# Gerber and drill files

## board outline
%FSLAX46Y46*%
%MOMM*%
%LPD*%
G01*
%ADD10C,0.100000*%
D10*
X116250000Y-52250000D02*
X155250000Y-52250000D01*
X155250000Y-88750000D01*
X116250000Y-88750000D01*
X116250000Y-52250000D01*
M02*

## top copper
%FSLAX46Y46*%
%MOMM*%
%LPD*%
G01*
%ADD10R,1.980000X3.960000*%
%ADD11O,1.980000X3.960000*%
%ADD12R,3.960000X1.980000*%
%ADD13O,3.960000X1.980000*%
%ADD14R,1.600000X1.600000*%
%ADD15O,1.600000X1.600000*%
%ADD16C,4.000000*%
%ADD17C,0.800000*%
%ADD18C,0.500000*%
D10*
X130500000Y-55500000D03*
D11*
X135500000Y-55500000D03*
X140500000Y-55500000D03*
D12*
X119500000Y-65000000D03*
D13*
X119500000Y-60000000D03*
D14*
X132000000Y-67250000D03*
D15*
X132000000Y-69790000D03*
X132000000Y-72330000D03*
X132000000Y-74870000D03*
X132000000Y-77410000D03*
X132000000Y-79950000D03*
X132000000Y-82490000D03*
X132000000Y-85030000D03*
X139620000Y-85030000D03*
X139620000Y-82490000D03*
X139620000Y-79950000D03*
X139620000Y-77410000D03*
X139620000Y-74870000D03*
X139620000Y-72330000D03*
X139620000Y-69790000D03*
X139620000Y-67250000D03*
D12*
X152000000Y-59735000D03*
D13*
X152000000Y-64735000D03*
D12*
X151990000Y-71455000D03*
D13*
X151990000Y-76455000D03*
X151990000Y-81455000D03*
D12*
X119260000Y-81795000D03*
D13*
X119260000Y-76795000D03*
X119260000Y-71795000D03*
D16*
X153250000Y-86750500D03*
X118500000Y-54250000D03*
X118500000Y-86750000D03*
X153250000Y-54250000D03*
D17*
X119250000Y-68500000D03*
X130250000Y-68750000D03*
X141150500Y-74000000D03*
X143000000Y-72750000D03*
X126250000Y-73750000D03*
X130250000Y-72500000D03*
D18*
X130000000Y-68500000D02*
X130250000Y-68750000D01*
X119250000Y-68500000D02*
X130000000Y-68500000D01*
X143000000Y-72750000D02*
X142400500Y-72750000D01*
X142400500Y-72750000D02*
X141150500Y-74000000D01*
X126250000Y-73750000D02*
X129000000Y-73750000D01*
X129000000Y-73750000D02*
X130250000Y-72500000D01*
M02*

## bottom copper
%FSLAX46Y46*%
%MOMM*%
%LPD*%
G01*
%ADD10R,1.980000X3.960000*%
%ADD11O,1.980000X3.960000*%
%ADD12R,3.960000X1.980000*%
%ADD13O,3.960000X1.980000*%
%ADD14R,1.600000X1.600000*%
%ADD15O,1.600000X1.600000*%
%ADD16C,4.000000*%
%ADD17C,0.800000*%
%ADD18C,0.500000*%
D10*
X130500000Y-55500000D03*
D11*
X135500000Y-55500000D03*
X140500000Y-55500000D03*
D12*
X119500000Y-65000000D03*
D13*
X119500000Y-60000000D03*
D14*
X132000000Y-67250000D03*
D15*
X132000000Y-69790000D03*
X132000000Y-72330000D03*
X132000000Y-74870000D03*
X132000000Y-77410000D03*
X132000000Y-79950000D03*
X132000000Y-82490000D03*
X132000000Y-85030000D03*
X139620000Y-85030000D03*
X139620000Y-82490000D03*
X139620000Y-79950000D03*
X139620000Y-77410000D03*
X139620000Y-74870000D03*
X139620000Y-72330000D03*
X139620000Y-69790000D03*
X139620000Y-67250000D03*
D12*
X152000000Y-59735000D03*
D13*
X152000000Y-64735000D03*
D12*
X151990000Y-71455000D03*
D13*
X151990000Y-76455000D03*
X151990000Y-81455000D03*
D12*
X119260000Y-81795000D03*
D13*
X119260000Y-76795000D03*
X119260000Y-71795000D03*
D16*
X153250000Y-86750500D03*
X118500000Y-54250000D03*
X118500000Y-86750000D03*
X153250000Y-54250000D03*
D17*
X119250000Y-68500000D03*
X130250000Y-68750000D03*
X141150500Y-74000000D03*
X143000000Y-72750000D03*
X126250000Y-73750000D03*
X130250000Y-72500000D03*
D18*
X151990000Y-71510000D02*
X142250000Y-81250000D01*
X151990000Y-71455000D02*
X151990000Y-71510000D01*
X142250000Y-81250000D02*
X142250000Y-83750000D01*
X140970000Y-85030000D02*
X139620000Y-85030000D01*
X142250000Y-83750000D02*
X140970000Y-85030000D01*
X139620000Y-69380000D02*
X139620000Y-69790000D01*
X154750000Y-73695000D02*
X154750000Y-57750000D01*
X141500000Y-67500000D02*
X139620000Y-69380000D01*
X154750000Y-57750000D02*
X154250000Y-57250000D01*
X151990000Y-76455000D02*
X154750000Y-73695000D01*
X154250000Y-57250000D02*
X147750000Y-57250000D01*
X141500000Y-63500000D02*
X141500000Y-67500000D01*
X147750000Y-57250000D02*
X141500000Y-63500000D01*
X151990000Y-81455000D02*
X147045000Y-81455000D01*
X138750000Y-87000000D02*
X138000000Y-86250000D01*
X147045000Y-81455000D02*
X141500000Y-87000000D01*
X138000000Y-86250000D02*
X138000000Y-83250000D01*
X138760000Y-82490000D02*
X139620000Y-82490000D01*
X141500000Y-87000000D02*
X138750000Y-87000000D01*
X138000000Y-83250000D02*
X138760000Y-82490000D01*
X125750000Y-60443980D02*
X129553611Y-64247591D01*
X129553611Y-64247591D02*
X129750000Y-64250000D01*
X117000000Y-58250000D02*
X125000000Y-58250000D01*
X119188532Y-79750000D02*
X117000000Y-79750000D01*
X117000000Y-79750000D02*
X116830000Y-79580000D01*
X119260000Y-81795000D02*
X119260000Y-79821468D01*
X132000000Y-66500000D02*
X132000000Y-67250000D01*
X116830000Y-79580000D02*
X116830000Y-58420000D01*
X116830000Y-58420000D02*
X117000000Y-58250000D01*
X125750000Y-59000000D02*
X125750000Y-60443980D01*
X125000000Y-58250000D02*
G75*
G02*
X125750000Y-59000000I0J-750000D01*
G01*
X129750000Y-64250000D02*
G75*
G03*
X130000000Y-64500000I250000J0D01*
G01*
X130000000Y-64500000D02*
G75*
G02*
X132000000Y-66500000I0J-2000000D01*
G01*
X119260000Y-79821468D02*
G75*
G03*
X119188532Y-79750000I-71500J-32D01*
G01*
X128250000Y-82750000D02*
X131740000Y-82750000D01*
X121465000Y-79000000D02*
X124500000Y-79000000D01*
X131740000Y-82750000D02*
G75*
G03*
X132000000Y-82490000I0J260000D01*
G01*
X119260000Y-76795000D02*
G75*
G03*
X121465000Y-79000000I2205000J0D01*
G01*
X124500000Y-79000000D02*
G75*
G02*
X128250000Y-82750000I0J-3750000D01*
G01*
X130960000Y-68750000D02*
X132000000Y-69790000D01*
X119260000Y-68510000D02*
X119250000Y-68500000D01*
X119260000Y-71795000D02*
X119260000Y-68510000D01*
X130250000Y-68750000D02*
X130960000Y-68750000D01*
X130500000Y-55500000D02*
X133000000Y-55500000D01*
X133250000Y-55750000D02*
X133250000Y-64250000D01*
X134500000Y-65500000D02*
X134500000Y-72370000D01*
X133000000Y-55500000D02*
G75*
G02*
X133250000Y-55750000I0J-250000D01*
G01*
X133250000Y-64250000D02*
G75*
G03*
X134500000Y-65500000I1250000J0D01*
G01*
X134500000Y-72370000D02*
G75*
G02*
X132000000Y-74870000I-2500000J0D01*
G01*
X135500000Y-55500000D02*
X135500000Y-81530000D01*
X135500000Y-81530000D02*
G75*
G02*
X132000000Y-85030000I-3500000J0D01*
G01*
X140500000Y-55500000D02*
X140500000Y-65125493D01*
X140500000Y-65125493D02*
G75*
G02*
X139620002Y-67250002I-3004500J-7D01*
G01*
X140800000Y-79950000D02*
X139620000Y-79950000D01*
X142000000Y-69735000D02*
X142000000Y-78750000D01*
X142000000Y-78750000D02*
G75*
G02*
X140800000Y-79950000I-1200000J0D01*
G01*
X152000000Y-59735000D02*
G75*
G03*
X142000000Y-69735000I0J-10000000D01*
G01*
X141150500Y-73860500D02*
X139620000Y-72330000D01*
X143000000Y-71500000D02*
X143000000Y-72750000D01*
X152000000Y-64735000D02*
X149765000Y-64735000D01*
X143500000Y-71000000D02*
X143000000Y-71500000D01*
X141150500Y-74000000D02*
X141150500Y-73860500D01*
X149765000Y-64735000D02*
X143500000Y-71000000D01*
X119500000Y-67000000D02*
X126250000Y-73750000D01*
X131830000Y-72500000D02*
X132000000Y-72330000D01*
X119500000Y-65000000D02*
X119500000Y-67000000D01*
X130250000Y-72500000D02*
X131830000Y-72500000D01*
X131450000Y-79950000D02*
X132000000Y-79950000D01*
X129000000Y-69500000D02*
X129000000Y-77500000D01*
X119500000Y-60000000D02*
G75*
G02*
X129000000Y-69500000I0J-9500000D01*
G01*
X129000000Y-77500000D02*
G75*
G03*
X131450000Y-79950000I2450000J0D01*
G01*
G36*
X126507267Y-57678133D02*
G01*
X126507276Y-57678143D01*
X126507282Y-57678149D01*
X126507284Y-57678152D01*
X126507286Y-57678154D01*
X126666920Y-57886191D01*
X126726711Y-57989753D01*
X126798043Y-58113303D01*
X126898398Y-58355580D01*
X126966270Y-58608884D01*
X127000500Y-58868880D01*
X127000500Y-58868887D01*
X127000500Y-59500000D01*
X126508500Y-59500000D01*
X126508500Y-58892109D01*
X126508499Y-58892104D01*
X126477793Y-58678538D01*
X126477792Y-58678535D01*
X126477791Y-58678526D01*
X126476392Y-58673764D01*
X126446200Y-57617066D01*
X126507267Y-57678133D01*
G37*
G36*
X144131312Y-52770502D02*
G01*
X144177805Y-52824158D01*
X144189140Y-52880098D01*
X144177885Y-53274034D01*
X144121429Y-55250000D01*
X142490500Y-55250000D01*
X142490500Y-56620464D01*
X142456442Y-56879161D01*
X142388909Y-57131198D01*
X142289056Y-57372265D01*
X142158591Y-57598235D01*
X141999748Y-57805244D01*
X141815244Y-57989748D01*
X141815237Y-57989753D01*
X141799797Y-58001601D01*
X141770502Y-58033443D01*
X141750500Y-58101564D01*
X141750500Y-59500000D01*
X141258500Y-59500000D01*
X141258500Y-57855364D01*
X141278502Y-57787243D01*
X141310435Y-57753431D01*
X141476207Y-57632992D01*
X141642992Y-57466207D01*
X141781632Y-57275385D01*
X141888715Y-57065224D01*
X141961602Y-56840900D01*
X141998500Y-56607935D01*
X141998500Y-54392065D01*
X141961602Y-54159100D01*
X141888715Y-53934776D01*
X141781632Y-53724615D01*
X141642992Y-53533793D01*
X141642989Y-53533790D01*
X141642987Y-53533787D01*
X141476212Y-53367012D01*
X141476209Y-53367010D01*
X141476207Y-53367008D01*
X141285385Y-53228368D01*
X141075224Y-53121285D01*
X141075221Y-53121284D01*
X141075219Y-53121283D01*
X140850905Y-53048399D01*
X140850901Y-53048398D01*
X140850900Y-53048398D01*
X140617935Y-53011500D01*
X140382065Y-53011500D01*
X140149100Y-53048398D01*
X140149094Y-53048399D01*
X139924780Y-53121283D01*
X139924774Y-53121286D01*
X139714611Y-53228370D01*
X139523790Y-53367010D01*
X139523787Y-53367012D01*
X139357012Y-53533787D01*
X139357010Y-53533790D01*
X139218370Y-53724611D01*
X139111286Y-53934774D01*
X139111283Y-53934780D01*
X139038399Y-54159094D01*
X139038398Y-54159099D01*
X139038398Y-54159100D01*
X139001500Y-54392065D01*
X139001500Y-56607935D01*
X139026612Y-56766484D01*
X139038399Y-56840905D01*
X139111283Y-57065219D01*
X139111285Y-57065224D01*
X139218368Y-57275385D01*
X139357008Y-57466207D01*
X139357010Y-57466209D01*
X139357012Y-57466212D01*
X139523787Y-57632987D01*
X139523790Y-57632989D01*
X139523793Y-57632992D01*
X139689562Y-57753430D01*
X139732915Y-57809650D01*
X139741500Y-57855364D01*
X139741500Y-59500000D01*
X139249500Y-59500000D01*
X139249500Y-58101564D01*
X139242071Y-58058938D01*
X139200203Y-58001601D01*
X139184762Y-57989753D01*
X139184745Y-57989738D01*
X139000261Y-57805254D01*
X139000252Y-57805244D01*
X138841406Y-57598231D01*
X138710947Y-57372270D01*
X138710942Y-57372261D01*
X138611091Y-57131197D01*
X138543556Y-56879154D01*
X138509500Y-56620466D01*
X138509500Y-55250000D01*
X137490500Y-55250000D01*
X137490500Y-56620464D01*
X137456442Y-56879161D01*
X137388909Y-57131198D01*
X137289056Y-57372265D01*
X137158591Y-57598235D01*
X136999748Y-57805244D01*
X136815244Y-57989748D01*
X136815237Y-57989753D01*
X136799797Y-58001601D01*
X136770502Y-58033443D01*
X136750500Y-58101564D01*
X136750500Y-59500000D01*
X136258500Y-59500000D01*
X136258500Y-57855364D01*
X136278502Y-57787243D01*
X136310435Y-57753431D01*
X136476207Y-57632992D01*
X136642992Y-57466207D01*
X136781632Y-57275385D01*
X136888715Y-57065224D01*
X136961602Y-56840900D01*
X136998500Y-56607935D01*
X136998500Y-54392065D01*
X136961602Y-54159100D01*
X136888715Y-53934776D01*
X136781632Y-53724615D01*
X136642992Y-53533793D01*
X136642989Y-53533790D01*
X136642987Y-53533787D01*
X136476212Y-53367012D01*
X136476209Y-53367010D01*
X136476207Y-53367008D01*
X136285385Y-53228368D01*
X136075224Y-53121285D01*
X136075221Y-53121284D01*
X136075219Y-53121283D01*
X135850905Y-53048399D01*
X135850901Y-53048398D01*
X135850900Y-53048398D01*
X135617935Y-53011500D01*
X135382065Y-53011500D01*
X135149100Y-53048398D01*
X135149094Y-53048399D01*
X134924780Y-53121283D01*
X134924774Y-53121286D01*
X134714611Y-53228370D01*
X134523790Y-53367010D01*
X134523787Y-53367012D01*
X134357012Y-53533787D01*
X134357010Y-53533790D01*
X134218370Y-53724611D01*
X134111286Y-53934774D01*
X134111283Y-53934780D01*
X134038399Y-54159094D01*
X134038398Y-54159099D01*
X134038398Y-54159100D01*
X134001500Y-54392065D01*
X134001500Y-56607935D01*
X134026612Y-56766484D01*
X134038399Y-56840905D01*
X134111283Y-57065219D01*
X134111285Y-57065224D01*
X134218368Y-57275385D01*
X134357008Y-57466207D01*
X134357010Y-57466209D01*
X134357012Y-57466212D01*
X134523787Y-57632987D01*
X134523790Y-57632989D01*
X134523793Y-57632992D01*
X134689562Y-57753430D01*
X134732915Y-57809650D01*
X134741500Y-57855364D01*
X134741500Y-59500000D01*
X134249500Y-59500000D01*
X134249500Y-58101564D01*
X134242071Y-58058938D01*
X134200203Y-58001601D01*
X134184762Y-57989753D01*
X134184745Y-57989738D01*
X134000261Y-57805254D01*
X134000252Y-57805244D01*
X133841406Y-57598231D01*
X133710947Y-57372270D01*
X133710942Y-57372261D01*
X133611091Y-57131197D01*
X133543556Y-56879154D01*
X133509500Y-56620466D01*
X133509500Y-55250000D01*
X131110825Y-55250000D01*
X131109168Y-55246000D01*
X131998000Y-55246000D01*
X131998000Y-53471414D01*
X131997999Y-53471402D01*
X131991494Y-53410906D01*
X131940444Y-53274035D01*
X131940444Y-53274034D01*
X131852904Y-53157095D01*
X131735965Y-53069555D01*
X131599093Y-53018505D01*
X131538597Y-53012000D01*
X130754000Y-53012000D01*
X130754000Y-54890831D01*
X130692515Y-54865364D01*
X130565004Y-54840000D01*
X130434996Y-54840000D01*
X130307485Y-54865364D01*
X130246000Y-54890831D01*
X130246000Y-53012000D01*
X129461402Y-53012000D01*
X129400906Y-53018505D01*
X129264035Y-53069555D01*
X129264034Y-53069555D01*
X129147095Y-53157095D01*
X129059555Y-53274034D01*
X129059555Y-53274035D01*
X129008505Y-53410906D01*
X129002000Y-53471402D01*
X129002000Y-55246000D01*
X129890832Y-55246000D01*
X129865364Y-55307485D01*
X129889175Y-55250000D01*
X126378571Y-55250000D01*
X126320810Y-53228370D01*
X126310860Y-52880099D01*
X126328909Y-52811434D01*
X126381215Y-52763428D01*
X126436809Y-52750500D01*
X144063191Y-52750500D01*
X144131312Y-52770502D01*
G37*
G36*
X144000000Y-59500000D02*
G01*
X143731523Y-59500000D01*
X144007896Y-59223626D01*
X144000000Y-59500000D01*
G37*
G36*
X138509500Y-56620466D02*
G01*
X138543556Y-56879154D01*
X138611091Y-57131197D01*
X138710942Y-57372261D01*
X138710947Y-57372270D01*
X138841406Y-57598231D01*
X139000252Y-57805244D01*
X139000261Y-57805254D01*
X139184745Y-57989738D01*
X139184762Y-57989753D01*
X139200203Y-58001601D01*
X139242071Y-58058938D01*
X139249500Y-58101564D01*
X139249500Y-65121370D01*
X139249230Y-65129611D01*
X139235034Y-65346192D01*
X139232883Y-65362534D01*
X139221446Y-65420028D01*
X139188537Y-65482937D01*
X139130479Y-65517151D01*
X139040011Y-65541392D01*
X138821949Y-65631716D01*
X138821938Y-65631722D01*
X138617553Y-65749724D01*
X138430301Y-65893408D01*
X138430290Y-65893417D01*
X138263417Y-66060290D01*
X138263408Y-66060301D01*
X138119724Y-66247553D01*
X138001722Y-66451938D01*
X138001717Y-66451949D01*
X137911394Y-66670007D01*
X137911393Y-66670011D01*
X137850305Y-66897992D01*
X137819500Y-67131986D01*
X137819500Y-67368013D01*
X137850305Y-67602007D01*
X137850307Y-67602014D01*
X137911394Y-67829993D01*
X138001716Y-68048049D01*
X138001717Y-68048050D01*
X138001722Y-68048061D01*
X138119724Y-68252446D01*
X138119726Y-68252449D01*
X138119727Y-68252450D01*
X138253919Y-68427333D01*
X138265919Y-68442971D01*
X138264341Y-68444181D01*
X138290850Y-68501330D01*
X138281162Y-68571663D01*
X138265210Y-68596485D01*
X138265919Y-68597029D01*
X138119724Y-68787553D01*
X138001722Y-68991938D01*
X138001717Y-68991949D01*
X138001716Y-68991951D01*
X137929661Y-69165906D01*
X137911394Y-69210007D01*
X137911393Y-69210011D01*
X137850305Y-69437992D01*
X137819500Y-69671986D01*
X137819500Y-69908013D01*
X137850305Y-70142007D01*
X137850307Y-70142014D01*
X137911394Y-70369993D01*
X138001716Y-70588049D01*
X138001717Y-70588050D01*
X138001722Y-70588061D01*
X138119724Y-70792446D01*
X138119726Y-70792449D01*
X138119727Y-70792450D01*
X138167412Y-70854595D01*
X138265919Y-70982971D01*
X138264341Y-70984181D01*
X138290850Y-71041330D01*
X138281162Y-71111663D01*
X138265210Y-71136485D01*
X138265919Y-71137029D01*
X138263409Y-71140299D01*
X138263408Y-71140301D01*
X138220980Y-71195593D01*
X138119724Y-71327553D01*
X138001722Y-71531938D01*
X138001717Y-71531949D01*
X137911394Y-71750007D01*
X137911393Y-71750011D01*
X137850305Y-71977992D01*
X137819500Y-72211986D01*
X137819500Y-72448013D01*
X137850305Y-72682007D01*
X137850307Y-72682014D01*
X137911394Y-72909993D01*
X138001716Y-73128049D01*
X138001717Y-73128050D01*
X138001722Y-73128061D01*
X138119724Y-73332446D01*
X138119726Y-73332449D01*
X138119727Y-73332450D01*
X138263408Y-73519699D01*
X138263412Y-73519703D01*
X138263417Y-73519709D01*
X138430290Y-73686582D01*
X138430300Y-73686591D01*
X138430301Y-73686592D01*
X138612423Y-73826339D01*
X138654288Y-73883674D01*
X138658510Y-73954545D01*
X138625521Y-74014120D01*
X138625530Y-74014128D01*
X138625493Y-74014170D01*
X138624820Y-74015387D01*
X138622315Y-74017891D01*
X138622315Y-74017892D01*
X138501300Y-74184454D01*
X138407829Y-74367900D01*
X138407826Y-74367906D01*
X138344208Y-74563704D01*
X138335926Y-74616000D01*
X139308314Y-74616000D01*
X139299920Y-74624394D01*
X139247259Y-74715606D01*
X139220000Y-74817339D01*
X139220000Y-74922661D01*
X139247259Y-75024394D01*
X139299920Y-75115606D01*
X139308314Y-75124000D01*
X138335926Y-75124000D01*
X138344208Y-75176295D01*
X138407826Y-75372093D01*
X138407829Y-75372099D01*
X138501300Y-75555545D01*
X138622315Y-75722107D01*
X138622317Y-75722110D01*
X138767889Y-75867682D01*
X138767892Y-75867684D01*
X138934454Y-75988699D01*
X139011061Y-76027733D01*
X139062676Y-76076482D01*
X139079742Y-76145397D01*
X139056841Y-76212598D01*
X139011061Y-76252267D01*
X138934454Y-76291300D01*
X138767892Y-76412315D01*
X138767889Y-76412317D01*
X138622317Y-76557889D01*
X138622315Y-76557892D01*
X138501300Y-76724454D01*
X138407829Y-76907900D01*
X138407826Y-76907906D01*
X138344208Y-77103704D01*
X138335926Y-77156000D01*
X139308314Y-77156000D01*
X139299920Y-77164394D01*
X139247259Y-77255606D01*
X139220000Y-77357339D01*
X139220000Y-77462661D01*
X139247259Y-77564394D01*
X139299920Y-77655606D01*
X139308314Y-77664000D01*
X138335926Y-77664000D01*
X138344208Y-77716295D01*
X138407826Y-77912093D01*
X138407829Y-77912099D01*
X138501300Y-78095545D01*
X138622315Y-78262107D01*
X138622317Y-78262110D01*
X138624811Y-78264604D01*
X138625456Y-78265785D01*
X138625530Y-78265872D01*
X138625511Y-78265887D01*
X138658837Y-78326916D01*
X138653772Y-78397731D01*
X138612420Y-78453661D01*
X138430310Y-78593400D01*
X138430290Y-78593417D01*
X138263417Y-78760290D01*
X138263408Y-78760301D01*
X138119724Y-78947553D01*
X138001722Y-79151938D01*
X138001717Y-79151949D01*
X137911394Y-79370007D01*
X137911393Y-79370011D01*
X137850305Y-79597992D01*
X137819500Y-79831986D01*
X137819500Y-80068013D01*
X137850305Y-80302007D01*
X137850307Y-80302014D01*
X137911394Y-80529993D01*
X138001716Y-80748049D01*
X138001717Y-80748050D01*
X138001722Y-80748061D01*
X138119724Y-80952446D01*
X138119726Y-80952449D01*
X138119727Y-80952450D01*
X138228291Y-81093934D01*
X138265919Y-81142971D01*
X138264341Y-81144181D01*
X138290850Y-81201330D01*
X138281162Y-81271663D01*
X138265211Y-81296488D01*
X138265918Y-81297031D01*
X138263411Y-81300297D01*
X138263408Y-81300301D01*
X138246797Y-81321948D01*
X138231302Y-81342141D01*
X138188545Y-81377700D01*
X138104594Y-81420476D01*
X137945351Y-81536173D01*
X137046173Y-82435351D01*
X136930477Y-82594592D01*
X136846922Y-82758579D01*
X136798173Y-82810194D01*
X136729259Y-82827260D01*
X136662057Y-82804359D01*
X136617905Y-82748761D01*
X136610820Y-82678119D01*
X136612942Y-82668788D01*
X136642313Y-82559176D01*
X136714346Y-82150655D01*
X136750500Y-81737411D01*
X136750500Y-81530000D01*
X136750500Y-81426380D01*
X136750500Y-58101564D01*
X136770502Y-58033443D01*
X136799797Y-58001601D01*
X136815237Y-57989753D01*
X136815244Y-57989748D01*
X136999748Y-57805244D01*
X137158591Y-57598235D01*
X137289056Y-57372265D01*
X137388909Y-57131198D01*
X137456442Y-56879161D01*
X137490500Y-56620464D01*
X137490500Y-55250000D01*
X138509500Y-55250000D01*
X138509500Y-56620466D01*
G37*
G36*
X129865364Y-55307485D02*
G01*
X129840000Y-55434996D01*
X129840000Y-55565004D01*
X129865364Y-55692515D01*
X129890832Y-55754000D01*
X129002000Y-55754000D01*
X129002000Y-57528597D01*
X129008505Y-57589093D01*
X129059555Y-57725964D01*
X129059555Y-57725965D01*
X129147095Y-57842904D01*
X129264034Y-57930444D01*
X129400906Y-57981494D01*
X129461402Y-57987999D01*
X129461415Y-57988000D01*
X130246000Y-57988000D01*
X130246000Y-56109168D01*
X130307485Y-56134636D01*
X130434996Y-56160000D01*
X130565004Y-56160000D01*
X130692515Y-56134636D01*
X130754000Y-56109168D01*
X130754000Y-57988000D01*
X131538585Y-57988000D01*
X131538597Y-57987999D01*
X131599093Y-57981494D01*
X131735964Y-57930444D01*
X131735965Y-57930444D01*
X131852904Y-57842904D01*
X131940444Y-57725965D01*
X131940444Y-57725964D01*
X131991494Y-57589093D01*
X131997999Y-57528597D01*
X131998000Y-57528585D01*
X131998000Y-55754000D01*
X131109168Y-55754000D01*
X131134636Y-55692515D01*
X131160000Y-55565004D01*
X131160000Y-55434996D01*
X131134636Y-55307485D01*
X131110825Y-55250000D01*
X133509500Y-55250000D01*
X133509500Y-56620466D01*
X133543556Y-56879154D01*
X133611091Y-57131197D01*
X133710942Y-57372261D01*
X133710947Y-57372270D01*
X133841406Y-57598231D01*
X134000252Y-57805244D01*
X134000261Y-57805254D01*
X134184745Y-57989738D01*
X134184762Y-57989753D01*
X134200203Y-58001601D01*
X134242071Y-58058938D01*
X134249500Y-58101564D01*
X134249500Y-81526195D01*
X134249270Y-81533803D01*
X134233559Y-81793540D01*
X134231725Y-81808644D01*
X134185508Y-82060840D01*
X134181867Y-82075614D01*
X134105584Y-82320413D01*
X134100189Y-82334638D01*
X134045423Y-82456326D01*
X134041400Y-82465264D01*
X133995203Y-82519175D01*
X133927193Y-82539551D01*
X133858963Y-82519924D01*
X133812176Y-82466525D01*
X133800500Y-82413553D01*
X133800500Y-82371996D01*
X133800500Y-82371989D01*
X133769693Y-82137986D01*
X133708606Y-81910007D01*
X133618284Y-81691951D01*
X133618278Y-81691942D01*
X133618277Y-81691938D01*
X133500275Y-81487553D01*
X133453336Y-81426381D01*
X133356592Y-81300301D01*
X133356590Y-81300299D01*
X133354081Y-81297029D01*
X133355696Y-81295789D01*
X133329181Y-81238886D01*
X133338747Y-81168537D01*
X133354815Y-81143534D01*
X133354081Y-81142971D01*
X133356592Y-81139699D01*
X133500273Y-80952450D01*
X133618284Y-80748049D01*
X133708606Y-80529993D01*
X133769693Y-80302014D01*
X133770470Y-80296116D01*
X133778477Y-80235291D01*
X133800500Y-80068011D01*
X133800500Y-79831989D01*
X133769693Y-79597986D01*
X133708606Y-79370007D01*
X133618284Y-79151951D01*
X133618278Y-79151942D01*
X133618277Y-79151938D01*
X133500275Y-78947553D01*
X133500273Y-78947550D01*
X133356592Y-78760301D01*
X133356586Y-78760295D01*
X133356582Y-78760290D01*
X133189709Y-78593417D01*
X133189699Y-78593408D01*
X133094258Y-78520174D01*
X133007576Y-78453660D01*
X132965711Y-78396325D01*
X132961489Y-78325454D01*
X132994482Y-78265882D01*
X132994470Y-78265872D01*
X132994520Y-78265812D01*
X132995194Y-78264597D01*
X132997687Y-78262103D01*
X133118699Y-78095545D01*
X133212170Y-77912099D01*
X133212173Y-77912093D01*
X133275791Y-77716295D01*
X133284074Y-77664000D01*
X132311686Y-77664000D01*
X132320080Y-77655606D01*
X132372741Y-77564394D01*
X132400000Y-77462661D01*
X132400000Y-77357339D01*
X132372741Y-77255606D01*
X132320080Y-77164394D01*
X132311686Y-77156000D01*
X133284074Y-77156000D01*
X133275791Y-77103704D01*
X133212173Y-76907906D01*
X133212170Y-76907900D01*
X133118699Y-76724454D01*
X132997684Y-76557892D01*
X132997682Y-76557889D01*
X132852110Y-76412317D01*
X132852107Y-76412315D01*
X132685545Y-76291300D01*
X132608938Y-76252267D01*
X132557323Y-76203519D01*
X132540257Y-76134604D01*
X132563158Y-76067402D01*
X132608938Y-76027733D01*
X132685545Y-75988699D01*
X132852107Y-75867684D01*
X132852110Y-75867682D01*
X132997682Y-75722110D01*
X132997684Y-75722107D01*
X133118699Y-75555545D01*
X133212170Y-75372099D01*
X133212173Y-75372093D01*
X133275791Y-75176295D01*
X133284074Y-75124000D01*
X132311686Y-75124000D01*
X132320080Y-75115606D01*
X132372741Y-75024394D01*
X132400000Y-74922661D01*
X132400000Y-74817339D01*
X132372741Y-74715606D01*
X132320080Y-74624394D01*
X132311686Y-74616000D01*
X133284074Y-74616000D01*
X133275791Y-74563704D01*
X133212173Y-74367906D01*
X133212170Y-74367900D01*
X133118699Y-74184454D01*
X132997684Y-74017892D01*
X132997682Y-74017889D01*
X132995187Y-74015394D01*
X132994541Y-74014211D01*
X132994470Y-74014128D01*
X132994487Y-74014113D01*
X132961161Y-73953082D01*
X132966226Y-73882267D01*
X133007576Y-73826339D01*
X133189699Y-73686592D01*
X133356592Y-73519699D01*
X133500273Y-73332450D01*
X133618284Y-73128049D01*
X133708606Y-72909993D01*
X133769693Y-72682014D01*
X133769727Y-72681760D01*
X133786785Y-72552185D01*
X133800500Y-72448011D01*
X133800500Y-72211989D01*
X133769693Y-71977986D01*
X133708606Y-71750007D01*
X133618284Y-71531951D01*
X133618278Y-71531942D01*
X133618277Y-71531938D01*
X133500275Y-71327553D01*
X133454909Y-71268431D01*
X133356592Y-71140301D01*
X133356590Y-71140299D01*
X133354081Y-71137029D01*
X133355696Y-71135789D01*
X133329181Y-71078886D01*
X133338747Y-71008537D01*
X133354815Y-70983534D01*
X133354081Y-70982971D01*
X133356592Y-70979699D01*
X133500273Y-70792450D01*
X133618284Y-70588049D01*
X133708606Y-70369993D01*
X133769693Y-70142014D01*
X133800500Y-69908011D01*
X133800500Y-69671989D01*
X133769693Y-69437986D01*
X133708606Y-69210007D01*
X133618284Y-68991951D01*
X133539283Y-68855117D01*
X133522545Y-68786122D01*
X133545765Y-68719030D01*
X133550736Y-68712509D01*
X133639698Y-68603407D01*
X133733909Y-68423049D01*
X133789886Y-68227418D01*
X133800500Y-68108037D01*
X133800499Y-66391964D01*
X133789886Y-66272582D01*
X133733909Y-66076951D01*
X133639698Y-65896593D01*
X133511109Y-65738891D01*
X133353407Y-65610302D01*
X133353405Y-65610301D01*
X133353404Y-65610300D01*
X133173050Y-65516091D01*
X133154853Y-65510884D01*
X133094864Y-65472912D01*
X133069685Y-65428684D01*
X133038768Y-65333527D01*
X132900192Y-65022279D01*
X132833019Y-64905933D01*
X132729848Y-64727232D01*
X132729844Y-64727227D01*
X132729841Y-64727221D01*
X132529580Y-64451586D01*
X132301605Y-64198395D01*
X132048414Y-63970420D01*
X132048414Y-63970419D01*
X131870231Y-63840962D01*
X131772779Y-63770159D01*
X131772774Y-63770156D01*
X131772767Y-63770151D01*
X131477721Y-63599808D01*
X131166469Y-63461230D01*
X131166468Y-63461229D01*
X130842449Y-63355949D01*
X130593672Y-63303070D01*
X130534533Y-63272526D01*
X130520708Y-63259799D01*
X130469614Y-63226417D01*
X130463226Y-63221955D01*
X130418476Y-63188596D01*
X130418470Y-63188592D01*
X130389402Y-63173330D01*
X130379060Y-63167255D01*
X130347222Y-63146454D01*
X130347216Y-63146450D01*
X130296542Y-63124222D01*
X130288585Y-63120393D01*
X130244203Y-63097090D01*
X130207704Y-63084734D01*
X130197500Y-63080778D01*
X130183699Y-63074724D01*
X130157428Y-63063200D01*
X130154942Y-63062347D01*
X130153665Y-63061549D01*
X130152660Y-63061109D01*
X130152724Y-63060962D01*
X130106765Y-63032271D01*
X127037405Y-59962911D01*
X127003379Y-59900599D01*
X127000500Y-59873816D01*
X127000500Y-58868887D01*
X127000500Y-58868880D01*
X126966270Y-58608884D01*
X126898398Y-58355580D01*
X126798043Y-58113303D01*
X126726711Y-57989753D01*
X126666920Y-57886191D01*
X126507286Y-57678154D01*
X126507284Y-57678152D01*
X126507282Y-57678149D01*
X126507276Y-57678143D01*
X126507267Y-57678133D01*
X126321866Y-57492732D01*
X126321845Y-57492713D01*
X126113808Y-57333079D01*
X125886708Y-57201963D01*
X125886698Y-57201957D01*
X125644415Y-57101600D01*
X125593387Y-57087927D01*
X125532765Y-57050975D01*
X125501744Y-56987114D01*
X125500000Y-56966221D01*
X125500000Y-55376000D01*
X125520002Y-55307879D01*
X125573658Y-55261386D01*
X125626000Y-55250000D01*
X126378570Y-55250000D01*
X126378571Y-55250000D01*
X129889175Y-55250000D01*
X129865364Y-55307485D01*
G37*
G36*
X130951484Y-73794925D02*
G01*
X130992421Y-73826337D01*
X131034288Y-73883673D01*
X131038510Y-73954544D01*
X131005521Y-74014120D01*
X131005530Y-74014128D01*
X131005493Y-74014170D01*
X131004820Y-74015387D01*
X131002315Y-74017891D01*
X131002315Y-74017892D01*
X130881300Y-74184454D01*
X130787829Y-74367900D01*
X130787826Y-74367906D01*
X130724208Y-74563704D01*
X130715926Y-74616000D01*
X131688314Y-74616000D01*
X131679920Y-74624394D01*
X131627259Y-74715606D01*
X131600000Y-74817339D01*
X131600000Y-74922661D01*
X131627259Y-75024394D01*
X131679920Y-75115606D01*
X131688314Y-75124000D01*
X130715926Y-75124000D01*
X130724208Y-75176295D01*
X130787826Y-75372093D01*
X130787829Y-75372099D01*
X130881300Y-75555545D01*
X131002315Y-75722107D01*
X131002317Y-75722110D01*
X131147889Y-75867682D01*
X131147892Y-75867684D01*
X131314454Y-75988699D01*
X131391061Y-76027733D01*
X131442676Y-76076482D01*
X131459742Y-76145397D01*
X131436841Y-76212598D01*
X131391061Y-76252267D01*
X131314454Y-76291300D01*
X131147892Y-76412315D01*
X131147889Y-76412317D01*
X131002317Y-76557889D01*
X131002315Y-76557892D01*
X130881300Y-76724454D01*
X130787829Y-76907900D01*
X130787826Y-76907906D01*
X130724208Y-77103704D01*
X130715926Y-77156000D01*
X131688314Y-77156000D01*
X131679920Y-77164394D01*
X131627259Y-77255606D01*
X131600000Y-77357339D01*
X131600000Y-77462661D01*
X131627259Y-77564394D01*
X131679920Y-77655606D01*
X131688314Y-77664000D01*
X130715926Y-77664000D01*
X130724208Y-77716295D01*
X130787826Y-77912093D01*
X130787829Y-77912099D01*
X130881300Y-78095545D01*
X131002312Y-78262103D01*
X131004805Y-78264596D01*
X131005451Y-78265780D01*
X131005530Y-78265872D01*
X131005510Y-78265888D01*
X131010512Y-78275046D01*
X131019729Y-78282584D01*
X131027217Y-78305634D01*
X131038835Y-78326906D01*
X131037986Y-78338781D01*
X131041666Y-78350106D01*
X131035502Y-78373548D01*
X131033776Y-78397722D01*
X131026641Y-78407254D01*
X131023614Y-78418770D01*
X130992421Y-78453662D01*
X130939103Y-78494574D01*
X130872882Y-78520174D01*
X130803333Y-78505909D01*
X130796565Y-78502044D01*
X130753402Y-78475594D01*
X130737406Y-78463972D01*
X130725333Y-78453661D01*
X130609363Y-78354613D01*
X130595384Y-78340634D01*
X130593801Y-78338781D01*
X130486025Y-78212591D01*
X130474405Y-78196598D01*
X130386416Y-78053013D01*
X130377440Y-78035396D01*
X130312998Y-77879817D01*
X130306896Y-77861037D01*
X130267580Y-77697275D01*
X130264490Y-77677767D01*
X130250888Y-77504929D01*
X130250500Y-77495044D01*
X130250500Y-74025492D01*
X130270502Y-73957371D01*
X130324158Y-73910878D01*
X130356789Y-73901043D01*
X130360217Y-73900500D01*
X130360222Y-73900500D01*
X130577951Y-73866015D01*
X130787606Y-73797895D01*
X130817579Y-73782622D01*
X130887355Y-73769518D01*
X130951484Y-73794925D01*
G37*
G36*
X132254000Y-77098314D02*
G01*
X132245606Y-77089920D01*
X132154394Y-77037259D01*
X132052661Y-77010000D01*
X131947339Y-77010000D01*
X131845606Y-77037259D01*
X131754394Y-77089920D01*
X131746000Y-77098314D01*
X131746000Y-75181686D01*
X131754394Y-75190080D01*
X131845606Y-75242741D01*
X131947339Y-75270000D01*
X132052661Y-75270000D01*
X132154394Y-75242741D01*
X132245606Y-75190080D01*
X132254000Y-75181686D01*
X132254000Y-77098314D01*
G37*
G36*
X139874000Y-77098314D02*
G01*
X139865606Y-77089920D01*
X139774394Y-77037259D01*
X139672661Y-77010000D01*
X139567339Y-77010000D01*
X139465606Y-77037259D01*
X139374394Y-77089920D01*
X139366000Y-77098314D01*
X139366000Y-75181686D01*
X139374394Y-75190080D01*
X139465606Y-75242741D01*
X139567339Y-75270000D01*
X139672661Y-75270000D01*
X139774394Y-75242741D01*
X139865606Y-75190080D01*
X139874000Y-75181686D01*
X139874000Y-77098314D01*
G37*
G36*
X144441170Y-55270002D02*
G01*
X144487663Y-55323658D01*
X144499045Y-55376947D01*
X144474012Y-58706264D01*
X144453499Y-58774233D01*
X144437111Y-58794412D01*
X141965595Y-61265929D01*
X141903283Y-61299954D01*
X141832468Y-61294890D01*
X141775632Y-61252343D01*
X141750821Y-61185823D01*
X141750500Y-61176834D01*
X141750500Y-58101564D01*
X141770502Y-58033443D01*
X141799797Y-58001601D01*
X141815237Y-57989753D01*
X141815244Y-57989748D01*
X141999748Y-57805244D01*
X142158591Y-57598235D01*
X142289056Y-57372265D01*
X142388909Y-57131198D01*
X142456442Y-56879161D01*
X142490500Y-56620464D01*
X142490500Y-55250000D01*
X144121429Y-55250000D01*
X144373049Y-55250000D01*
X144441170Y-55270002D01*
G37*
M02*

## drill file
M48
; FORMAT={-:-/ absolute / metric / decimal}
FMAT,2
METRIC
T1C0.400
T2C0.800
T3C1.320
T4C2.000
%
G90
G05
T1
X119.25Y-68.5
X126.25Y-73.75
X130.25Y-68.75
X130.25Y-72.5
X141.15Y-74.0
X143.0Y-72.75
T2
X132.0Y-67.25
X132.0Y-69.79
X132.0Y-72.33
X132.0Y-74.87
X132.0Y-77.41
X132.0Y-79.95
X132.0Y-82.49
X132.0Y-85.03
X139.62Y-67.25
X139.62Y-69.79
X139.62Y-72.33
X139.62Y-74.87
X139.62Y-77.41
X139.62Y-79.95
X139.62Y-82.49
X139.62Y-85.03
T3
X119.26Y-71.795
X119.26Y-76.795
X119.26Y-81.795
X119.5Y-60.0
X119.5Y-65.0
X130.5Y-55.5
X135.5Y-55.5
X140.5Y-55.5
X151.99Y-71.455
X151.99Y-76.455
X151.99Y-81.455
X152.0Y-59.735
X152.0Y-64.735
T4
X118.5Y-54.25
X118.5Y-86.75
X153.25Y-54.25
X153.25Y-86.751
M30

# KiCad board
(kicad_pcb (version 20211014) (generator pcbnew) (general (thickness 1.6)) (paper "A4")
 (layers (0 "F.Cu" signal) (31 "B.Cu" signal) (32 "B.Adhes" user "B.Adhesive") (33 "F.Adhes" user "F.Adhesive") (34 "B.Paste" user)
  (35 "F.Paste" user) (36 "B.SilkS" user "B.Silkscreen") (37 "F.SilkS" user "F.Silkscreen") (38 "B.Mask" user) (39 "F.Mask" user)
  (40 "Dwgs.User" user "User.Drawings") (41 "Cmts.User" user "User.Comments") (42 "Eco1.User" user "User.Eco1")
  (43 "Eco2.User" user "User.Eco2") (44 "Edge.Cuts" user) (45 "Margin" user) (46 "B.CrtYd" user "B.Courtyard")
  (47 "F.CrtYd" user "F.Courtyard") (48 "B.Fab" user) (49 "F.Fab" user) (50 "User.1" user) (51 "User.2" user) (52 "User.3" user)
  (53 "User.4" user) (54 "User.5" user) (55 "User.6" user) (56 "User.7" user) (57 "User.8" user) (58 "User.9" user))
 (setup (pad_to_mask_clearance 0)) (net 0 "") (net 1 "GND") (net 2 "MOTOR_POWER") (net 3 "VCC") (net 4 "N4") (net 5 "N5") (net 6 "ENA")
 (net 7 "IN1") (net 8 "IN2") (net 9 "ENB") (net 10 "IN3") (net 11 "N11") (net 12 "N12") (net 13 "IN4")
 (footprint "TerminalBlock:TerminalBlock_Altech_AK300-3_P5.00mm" (layer "F.Cu") (at 130.5 55.5)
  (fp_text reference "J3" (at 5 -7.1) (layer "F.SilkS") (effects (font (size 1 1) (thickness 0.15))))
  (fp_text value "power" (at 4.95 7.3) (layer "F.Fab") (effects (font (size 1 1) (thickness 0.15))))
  (pad "1" thru_hole rect (at 0 0) (size 1.98 3.96) (drill 1.32) (layers *.Cu *.Mask) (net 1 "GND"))
  (pad "2" thru_hole oval (at 5 0) (size 1.98 3.96) (drill 1.32) (layers *.Cu *.Mask) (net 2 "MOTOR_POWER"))
  (pad "3" thru_hole oval (at 10 0) (size 1.98 3.96) (drill 1.32) (layers *.Cu *.Mask) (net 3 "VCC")))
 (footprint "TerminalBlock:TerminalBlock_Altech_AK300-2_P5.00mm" (layer "F.Cu") (at 119.5 65 90)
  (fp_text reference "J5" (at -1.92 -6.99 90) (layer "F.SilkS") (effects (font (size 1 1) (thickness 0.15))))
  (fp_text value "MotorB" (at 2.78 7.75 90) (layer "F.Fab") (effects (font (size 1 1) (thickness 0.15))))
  (pad "1" thru_hole rect (at 0 0 90) (size 1.98 3.96) (drill 1.32) (layers *.Cu *.Mask) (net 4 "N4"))
  (pad "2" thru_hole oval (at 5 0 90) (size 1.98 3.96) (drill 1.32) (layers *.Cu *.Mask) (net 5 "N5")))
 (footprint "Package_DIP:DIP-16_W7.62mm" (layer "F.Cu") (at 132 67.25)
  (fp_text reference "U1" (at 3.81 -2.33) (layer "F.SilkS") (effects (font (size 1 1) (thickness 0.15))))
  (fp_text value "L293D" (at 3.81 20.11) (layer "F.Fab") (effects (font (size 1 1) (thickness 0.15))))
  (pad "1" thru_hole rect (at 0 0) (size 1.6 1.6) (drill 0.8) (layers *.Cu *.Mask) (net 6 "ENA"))
  (pad "2" thru_hole oval (at 0 2.54) (size 1.6 1.6) (drill 0.8) (layers *.Cu *.Mask) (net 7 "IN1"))
  (pad "3" thru_hole oval (at 0 5.08) (size 1.6 1.6) (drill 0.8) (layers *.Cu *.Mask) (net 4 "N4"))
  (pad "4" thru_hole oval (at 0 7.62) (size 1.6 1.6) (drill 0.8) (layers *.Cu *.Mask) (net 1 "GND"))
  (pad "5" thru_hole oval (at 0 10.16) (size 1.6 1.6) (drill 0.8) (layers *.Cu *.Mask) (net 1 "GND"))
  (pad "6" thru_hole oval (at 0 12.7) (size 1.6 1.6) (drill 0.8) (layers *.Cu *.Mask) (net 5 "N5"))
  (pad "7" thru_hole oval (at 0 15.24) (size 1.6 1.6) (drill 0.8) (layers *.Cu *.Mask) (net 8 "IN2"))
  (pad "8" thru_hole oval (at 0 17.78) (size 1.6 1.6) (drill 0.8) (layers *.Cu *.Mask) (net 2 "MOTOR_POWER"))
  (pad "9" thru_hole oval (at 7.62 17.78) (size 1.6 1.6) (drill 0.8) (layers *.Cu *.Mask) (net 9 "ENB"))
  (pad "10" thru_hole oval (at 7.62 15.24) (size 1.6 1.6) (drill 0.8) (layers *.Cu *.Mask) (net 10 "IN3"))
  (pad "11" thru_hole oval (at 7.62 12.7) (size 1.6 1.6) (drill 0.8) (layers *.Cu *.Mask) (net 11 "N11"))
  (pad "12" thru_hole oval (at 7.62 10.16) (size 1.6 1.6) (drill 0.8) (layers *.Cu *.Mask) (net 1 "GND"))
  (pad "13" thru_hole oval (at 7.62 7.62) (size 1.6 1.6) (drill 0.8) (layers *.Cu *.Mask) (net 1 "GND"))
  (pad "14" thru_hole oval (at 7.62 5.08) (size 1.6 1.6) (drill 0.8) (layers *.Cu *.Mask) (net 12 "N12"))
  (pad "15" thru_hole oval (at 7.62 2.54) (size 1.6 1.6) (drill 0.8) (layers *.Cu *.Mask) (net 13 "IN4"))
  (pad "16" thru_hole oval (at 7.62 0) (size 1.6 1.6) (drill 0.8) (layers *.Cu *.Mask) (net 3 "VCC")))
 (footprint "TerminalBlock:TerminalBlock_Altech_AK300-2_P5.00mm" (layer "F.Cu") (at 152 59.735 -90)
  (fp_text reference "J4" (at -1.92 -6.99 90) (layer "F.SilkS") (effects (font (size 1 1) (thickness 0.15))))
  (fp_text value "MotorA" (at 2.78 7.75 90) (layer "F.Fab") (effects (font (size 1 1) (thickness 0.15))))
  (pad "1" thru_hole rect (at 0 0 270) (size 1.98 3.96) (drill 1.32) (layers *.Cu *.Mask) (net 11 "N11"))
  (pad "2" thru_hole oval (at 5 0 270) (size 1.98 3.96) (drill 1.32) (layers *.Cu *.Mask) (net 12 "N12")))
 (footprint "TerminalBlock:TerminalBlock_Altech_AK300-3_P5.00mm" (layer "F.Cu") (at 151.99 71.455 -90)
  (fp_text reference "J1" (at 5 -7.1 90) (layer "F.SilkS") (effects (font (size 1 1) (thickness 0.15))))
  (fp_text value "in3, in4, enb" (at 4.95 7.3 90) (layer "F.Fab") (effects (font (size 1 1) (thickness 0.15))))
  (pad "1" thru_hole rect (at 0 0 270) (size 1.98 3.96) (drill 1.32) (layers *.Cu *.Mask) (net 9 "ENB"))
  (pad "2" thru_hole oval (at 5 0 270) (size 1.98 3.96) (drill 1.32) (layers *.Cu *.Mask) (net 13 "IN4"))
  (pad "3" thru_hole oval (at 10 0 270) (size 1.98 3.96) (drill 1.32) (layers *.Cu *.Mask) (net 10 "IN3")))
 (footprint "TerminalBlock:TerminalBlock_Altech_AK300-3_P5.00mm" (layer "F.Cu") (at 119.26 81.795 90)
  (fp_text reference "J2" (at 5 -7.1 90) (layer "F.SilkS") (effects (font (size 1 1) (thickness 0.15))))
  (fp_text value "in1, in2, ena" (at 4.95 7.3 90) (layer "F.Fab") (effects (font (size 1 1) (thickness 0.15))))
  (pad "1" thru_hole rect (at 0 0 90) (size 1.98 3.96) (drill 1.32) (layers *.Cu *.Mask) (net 6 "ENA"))
  (pad "2" thru_hole oval (at 5 0 90) (size 1.98 3.96) (drill 1.32) (layers *.Cu *.Mask) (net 8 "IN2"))
  (pad "3" thru_hole oval (at 10 0 90) (size 1.98 3.96) (drill 1.32) (layers *.Cu *.Mask) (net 7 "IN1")))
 (gr_rect (start 116.25 52.25) (end 155.25 88.75) (layer "Edge.Cuts") (width 0.1) (fill none))
 (via (at 153.25 86.7505) (size 4) (drill 2) (layers "F.Cu" "B.Cu") (free) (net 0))
 (via (at 118.5 54.25) (size 4) (drill 2) (layers "F.Cu" "B.Cu") (free) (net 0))
 (via (at 118.5 86.75) (size 4) (drill 2) (layers "F.Cu" "B.Cu") (free) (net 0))
 (via (at 153.25 54.25) (size 4) (drill 2) (layers "F.Cu" "B.Cu") (free) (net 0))
 (segment (start 151.99 71.51) (end 142.25 81.25) (width 0.5) (layer "B.Cu") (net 9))
 (segment (start 151.99 71.455) (end 151.99 71.51) (width 0.5) (layer "B.Cu") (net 9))
 (segment (start 142.25 81.25) (end 142.25 83.75) (width 0.5) (layer "B.Cu") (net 9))
 (segment (start 140.97 85.03) (end 139.62 85.03) (width 0.5) (layer "B.Cu") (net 9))
 (segment (start 142.25 83.75) (end 140.97 85.03) (width 0.5) (layer "B.Cu") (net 9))
 (segment (start 139.62 69.38) (end 139.62 69.79) (width 0.5) (layer "B.Cu") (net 13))
 (segment (start 154.75 73.695) (end 154.75 57.75) (width 0.5) (layer "B.Cu") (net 13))
 (segment (start 141.5 67.5) (end 139.62 69.38) (width 0.5) (layer "B.Cu") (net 13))
 (segment (start 154.75 57.75) (end 154.25 57.25) (width 0.5) (layer "B.Cu") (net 13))
 (segment (start 151.99 76.455) (end 154.75 73.695) (width 0.5) (layer "B.Cu") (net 13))
 (segment (start 154.25 57.25) (end 147.75 57.25) (width 0.5) (layer "B.Cu") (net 13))
 (segment (start 141.5 63.5) (end 141.5 67.5) (width 0.5) (layer "B.Cu") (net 13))
 (segment (start 147.75 57.25) (end 141.5 63.5) (width 0.5) (layer "B.Cu") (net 13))
 (segment (start 151.99 81.455) (end 147.045 81.455) (width 0.5) (layer "B.Cu") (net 10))
 (segment (start 138.75 87) (end 138 86.25) (width 0.5) (layer "B.Cu") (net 10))
 (segment (start 147.045 81.455) (end 141.5 87) (width 0.5) (layer "B.Cu") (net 10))
 (segment (start 138 86.25) (end 138 83.25) (width 0.5) (layer "B.Cu") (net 10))
 (segment (start 138.76 82.49) (end 139.62 82.49) (width 0.5) (layer "B.Cu") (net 10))
 (segment (start 141.5 87) (end 138.75 87) (width 0.5) (layer "B.Cu") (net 10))
 (segment (start 138 83.25) (end 138.76 82.49) (width 0.5) (layer "B.Cu") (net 10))
 (segment (start 125.75 60.44398) (end 129.553611 64.247591) (width 0.5) (layer "B.Cu") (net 6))
 (segment (start 129.553611 64.247591) (end 129.75 64.25) (width 0.5) (layer "B.Cu") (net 6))
 (segment (start 117 58.25) (end 125 58.25) (width 0.5) (layer "B.Cu") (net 6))
 (segment (start 119.188532 79.75) (end 117 79.75) (width 0.5) (layer "B.Cu") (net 6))
 (segment (start 117 79.75) (end 116.83 79.58) (width 0.5) (layer "B.Cu") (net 6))
 (segment (start 119.26 81.795) (end 119.26 79.821468) (width 0.5) (layer "B.Cu") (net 6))
 (segment (start 132 66.5) (end 132 67.25) (width 0.5) (layer "B.Cu") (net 6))
 (segment (start 116.83 79.58) (end 116.83 58.42) (width 0.5) (layer "B.Cu") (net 6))
 (segment (start 116.83 58.42) (end 117 58.25) (width 0.5) (layer "B.Cu") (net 6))
 (segment (start 125.75 59) (end 125.75 60.44398) (width 0.5) (layer "B.Cu") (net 6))
 (arc (start 125 58.25) (mid 125.53033 58.46967) (end 125.75 59) (width 0.5) (layer "B.Cu") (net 6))
 (arc (start 129.75 64.25) (mid 129.823223 64.426777) (end 130 64.5) (width 0.5) (layer "B.Cu") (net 6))
 (arc (start 130 64.5) (mid 131.414214 65.085786) (end 132 66.5) (width 0.5) (layer "B.Cu") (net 6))
 (arc (start 119.26 79.821468) (mid 119.239068 79.770932) (end 119.188532 79.75) (width 0.5) (layer "B.Cu") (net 6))
 (segment (start 128.25 82.75) (end 131.74 82.75) (width 0.5) (layer "B.Cu") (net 8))
 (segment (start 121.465 79) (end 124.5 79) (width 0.5) (layer "B.Cu") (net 8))
 (arc (start 131.74 82.75) (mid 131.923848 82.673848) (end 132 82.49) (width 0.5) (layer "B.Cu") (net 8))
 (arc (start 119.26 76.795) (mid 119.90583 78.35417) (end 121.465 79) (width 0.5) (layer "B.Cu") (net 8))
 (arc (start 124.5 79) (mid 127.15165 80.09835) (end 128.25 82.75) (width 0.5) (layer "B.Cu") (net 8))
 (segment (start 130 68.5) (end 130.25 68.75) (width 0.5) (layer "F.Cu") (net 7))
 (segment (start 119.25 68.5) (end 130 68.5) (width 0.5) (layer "F.Cu") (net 7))
 (via (at 119.25 68.5) (size 0.8) (drill 0.4) (layers "F.Cu" "B.Cu") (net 7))
 (via (at 130.25 68.75) (size 0.8) (drill 0.4) (layers "F.Cu" "B.Cu") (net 7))
 (segment (start 130.96 68.75) (end 132 69.79) (width 0.5) (layer "B.Cu") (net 7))
 (segment (start 119.26 68.51) (end 119.25 68.5) (width 0.5) (layer "B.Cu") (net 7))
 (segment (start 119.26 71.795) (end 119.26 68.51) (width 0.5) (layer "B.Cu") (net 7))
 (segment (start 130.25 68.75) (end 130.96 68.75) (width 0.5) (layer "B.Cu") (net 7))
 (segment (start 130.5 55.5) (end 133 55.5) (width 0.5) (layer "B.Cu") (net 1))
 (segment (start 133.25 55.75) (end 133.25 64.25) (width 0.5) (layer "B.Cu") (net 1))
 (segment (start 134.5 65.5) (end 134.5 72.37) (width 0.5) (layer "B.Cu") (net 1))
 (arc (start 133 55.5) (mid 133.176777 55.573223) (end 133.25 55.75) (width 0.5) (layer "B.Cu") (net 1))
 (arc (start 133.25 64.25) (mid 133.616117 65.133883) (end 134.5 65.5) (width 0.5) (layer "B.Cu") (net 1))
 (arc (start 134.5 72.37) (mid 133.767767 74.137767) (end 132 74.87) (width 0.5) (layer "B.Cu") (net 1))
 (segment (start 135.5 55.5) (end 135.5 81.53) (width 0.5) (layer "B.Cu") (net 2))
 (arc (start 135.5 81.53) (mid 134.474874 84.004874) (end 132 85.03) (width 0.5) (layer "B.Cu") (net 2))
 (segment (start 140.5 55.5) (end 140.5 65.125493) (width 0.5) (layer "B.Cu") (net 3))
 (arc (start 140.5 65.125493) (mid 140.271295 66.275268) (end 139.62 67.25) (width 0.5) (layer "B.Cu") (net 3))
 (segment (start 140.8 79.95) (end 139.62 79.95) (width 0.5) (layer "B.Cu") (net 11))
 (segment (start 142 69.735) (end 142 78.75) (width 0.5) (layer "B.Cu") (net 11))
 (arc (start 142 78.75) (mid 141.648528 79.598528) (end 140.8 79.95) (width 0.5) (layer "B.Cu") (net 11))
 (arc (start 152 59.735) (mid 144.928932 62.663932) (end 142 69.735) (width 0.5) (layer "B.Cu") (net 11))
 (segment (start 143 72.75) (end 142.4005 72.75) (width 0.5) (layer "F.Cu") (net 12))
 (segment (start 142.4005 72.75) (end 141.1505 74) (width 0.5) (layer "F.Cu") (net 12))
 (via (at 141.1505 74) (size 0.8) (drill 0.4) (layers "F.Cu" "B.Cu") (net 12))
 (via (at 143 72.75) (size 0.8) (drill 0.4) (layers "F.Cu" "B.Cu") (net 12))
 (segment (start 141.1505 73.8605) (end 139.62 72.33) (width 0.5) (layer "B.Cu") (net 12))
 (segment (start 143 71.5) (end 143 72.75) (width 0.5) (layer "B.Cu") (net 12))
 (segment (start 152 64.735) (end 149.765 64.735) (width 0.5) (layer "B.Cu") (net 12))
 (segment (start 143.5 71) (end 143 71.5) (width 0.5) (layer "B.Cu") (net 12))
 (segment (start 141.1505 74) (end 141.1505 73.8605) (width 0.5) (layer "B.Cu") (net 12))
 (segment (start 149.765 64.735) (end 143.5 71) (width 0.5) (layer "B.Cu") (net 12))
 (segment (start 126.25 73.75) (end 129 73.75) (width 0.5) (layer "F.Cu") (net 4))
 (segment (start 129 73.75) (end 130.25 72.5) (width 0.5) (layer "F.Cu") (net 4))
 (via (at 126.25 73.75) (size 0.8) (drill 0.4) (layers "F.Cu" "B.Cu") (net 4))
 (via (at 130.25 72.5) (size 0.8) (drill 0.4) (layers "F.Cu" "B.Cu") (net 4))
 (segment (start 119.5 67) (end 126.25 73.75) (width 0.5) (layer "B.Cu") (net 4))
 (segment (start 131.83 72.5) (end 132 72.33) (width 0.5) (layer "B.Cu") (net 4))
 (segment (start 119.5 65) (end 119.5 67) (width 0.5) (layer "B.Cu") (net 4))
 (segment (start 130.25 72.5) (end 131.83 72.5) (width 0.5) (layer "B.Cu") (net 4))
 (segment (start 131.45 79.95) (end 132 79.95) (width 0.5) (layer "B.Cu") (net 5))
 (segment (start 129 69.5) (end 129 77.5) (width 0.5) (layer "B.Cu") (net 5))
 (arc (start 119.5 60) (mid 126.217514 62.782486) (end 129 69.5) (width 0.5) (layer "B.Cu") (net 5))
 (arc (start 129 77.5) (mid 129.717588 79.232412) (end 131.45 79.95) (width 0.5) (layer "B.Cu") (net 5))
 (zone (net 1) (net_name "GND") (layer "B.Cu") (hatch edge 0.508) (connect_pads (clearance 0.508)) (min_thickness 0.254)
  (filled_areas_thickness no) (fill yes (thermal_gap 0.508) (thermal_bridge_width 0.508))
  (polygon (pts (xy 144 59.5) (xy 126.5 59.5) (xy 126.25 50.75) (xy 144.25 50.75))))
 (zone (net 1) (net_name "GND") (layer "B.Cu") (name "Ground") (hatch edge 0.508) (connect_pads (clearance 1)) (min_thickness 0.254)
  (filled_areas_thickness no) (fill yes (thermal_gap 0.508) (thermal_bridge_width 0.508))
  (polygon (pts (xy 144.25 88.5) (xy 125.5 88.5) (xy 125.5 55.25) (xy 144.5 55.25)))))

